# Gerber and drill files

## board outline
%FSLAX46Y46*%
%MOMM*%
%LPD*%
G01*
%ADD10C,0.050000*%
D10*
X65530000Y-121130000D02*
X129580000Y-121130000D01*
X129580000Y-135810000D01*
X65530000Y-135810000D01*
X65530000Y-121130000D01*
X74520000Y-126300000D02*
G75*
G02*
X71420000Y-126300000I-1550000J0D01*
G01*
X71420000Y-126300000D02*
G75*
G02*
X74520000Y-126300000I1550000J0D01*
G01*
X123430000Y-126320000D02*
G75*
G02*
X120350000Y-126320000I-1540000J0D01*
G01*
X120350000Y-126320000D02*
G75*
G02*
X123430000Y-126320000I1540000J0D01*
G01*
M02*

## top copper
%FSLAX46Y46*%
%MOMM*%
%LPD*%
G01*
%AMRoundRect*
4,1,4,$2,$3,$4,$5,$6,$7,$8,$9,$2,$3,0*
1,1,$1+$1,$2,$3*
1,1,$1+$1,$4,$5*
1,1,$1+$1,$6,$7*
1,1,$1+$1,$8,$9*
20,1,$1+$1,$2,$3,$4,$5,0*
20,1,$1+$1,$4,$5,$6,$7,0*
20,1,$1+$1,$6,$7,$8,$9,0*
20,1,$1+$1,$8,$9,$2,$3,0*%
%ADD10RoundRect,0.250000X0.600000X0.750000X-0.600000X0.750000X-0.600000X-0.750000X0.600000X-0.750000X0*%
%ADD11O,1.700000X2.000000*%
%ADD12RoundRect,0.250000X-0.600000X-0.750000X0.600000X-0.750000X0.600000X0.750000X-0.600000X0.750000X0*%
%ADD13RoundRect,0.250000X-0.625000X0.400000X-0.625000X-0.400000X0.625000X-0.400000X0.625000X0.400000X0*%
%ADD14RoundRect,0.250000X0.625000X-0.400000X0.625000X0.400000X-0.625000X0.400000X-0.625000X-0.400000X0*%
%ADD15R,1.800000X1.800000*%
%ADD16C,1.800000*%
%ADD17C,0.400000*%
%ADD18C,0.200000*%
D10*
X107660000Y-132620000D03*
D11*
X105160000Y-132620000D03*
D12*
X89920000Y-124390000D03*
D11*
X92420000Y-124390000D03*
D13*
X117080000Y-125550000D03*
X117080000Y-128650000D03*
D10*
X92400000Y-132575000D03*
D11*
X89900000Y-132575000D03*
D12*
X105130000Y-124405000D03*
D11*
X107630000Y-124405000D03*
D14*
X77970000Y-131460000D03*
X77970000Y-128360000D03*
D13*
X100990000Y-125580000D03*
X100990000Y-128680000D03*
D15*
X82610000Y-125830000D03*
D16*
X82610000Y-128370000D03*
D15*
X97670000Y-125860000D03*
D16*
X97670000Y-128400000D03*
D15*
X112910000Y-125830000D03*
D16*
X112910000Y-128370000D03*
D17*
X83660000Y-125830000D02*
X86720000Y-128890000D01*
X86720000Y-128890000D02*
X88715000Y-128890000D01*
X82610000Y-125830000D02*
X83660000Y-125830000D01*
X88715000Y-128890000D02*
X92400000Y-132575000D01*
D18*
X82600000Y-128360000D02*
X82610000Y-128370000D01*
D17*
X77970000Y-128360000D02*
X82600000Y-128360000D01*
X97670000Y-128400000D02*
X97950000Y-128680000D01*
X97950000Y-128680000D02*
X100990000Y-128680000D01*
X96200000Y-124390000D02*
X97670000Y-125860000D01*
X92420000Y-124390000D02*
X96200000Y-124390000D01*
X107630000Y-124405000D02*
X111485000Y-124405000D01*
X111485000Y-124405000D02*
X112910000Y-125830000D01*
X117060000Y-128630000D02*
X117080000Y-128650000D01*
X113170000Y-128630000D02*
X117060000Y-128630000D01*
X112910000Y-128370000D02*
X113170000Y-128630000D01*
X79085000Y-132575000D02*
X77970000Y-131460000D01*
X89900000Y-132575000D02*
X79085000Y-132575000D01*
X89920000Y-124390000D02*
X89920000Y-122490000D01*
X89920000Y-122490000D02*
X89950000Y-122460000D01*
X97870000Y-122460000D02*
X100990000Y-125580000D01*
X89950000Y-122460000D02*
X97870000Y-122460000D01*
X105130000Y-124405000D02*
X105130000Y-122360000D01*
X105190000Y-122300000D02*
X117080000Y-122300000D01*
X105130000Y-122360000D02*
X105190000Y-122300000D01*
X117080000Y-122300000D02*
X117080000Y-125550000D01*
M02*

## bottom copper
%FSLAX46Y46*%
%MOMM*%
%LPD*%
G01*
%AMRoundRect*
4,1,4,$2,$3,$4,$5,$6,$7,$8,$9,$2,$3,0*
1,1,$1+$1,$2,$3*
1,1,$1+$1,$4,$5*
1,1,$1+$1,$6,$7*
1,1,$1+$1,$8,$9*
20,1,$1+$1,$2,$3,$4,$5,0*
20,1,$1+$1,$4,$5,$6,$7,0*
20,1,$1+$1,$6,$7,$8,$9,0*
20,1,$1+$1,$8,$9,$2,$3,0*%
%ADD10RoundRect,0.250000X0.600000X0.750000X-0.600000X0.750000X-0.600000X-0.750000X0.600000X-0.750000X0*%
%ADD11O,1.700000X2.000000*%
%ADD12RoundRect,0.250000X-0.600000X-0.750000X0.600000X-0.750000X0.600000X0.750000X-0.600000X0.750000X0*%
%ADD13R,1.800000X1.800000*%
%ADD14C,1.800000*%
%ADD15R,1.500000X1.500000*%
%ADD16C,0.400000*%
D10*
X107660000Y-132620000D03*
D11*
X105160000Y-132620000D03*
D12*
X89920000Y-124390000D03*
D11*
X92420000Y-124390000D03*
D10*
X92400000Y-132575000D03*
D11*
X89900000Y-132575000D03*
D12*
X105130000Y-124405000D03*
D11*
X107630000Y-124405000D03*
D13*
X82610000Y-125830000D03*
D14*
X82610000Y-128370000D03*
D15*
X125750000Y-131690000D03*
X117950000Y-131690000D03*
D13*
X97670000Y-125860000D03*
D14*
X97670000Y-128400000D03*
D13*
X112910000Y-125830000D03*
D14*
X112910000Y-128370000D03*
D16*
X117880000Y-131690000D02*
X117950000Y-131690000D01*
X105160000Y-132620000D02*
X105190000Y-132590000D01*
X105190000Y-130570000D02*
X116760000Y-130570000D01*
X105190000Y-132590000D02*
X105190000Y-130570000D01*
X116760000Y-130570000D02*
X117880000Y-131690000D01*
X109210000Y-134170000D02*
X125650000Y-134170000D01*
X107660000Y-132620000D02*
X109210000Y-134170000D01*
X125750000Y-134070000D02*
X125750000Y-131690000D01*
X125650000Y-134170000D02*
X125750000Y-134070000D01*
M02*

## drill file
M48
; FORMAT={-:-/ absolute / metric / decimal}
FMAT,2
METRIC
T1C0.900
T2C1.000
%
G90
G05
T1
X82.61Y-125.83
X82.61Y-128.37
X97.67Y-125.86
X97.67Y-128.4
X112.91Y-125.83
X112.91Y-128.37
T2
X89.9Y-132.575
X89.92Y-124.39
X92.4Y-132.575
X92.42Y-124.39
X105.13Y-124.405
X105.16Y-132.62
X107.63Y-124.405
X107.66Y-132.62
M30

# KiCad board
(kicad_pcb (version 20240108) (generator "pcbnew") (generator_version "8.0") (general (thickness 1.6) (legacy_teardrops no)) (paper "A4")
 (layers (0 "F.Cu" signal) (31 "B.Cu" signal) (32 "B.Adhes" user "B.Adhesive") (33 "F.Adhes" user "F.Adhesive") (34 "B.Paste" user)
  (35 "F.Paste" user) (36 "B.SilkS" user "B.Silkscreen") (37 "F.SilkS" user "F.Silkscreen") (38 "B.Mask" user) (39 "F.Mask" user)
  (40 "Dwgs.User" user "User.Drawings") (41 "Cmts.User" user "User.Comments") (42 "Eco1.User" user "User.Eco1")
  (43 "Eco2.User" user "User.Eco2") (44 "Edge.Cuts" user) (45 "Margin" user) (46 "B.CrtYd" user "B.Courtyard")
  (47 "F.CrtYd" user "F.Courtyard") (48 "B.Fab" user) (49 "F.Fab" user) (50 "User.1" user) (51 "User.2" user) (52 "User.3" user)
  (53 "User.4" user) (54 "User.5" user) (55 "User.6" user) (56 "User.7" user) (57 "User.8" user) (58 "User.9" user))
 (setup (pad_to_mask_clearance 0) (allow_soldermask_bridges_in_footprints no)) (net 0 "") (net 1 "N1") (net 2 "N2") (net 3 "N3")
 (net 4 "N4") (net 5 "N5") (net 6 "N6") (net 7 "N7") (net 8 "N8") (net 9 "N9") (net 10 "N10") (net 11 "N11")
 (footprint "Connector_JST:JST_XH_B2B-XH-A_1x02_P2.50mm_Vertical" (layer "F.Cu") (at 107.66 132.62 180)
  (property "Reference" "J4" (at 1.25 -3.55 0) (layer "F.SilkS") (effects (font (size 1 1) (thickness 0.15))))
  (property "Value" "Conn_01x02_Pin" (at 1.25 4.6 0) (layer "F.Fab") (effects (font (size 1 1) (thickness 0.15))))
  (pad "1" thru_hole roundrect (at 0 0 180) (size 1.7 2) (drill 1) (layers "*.Cu" "*.Mask") (remove_unused_layers no)
   (roundrect_rratio 0.147059) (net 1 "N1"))
  (pad "2" thru_hole oval (at 2.5 0 180) (size 1.7 2) (drill 1) (layers "*.Cu" "*.Mask") (remove_unused_layers no) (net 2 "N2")))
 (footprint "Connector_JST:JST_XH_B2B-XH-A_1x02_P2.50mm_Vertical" (layer "F.Cu") (at 89.92 124.39)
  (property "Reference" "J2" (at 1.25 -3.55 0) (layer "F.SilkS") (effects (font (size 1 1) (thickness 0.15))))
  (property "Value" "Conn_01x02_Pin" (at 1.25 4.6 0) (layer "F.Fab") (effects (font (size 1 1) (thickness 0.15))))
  (pad "1" thru_hole roundrect (at 0 0) (size 1.7 2) (drill 1) (layers "*.Cu" "*.Mask") (remove_unused_layers no)
   (roundrect_rratio 0.147059) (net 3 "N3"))
  (pad "2" thru_hole oval (at 2.5 0) (size 1.7 2) (drill 1) (layers "*.Cu" "*.Mask") (remove_unused_layers no) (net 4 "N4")))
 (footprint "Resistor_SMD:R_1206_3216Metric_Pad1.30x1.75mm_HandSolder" (layer "F.Cu") (at 117.08 127.1 -90)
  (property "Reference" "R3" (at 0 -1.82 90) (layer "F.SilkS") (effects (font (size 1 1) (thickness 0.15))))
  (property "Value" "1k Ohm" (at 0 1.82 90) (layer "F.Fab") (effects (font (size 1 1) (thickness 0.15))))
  (pad "1" smd roundrect (at -1.55 0 270) (size 1.3 1.75) (layers "F.Cu" "F.Paste" "F.Mask") (roundrect_rratio 0.192308) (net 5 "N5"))
  (pad "2" smd roundrect (at 1.55 0 270) (size 1.3 1.75) (layers "F.Cu" "F.Paste" "F.Mask") (roundrect_rratio 0.192308) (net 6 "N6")))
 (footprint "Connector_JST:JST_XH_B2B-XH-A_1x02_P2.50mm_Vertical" (layer "F.Cu") (at 92.4 132.575 180)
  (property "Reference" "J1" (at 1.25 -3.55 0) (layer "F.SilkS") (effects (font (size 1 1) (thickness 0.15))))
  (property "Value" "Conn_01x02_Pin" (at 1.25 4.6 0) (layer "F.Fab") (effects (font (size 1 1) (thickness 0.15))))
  (pad "1" thru_hole roundrect (at 0 0 180) (size 1.7 2) (drill 1) (layers "*.Cu" "*.Mask") (remove_unused_layers no)
   (roundrect_rratio 0.147059) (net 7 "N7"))
  (pad "2" thru_hole oval (at 2.5 0 180) (size 1.7 2) (drill 1) (layers "*.Cu" "*.Mask") (remove_unused_layers no) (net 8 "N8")))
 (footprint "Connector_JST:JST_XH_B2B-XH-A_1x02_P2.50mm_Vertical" (layer "F.Cu") (at 105.13 124.405)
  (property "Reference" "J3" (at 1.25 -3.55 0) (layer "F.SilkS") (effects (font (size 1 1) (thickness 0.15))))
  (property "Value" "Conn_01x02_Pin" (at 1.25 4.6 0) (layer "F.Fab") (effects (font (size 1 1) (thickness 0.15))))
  (pad "1" thru_hole roundrect (at 0 0) (size 1.7 2) (drill 1) (layers "*.Cu" "*.Mask") (remove_unused_layers no)
   (roundrect_rratio 0.147059) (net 5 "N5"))
  (pad "2" thru_hole oval (at 2.5 0) (size 1.7 2) (drill 1) (layers "*.Cu" "*.Mask") (remove_unused_layers no) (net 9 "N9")))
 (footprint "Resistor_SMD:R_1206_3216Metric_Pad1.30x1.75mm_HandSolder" (layer "F.Cu") (at 77.97 129.91 90)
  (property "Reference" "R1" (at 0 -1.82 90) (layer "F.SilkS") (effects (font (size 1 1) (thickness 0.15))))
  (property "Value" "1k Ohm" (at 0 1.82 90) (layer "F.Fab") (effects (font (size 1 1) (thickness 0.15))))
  (pad "1" smd roundrect (at -1.55 0 90) (size 1.3 1.75) (layers "F.Cu" "F.Paste" "F.Mask") (roundrect_rratio 0.192308) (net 8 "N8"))
  (pad "2" smd roundrect (at 1.55 0 90) (size 1.3 1.75) (layers "F.Cu" "F.Paste" "F.Mask") (roundrect_rratio 0.192308) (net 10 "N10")))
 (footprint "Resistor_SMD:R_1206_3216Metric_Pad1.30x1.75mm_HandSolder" (layer "F.Cu") (at 100.99 127.13 -90)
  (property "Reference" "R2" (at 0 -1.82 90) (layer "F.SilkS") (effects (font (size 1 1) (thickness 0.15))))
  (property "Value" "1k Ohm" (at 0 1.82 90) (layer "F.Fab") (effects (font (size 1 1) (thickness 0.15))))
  (pad "1" smd roundrect (at -1.55 0 270) (size 1.3 1.75) (layers "F.Cu" "F.Paste" "F.Mask") (roundrect_rratio 0.192308) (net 3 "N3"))
  (pad "2" smd roundrect (at 1.55 0 270) (size 1.3 1.75) (layers "F.Cu" "F.Paste" "F.Mask") (roundrect_rratio 0.192308) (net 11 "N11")))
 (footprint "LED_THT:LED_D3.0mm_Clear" (layer "B.Cu") (at 82.61 125.83 -90)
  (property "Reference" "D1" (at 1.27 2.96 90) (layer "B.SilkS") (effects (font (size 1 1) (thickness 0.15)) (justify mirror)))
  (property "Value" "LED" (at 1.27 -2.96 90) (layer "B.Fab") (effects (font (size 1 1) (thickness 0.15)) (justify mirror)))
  (pad "1" thru_hole rect (at 0 0 270) (size 1.8 1.8) (drill 0.9) (layers "*.Cu" "*.Mask") (remove_unused_layers no) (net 7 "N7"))
  (pad "2" thru_hole circle (at 2.54 0 270) (size 1.8 1.8) (drill 0.9) (layers "*.Cu" "*.Mask") (remove_unused_layers no) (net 10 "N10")))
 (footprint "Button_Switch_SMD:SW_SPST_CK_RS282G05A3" (layer "B.Cu") (at 121.85 131.69 180)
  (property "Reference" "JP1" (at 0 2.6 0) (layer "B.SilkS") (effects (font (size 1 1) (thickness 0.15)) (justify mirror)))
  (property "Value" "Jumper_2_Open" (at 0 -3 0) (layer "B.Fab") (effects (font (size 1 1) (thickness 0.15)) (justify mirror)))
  (pad "1" smd rect (at -3.9 0 180) (size 1.5 1.5) (layers "B.Cu" "B.Paste" "B.Mask") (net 1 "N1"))
  (pad "2" smd rect (at 3.9 0 180) (size 1.5 1.5) (layers "B.Cu" "B.Paste" "B.Mask") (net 2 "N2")))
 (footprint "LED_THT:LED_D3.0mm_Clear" (layer "B.Cu") (at 97.67 125.86 -90)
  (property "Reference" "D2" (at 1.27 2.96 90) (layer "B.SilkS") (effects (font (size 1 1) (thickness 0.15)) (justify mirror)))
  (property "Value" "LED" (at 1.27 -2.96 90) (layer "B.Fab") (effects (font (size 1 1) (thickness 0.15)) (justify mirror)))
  (pad "1" thru_hole rect (at 0 0 270) (size 1.8 1.8) (drill 0.9) (layers "*.Cu" "*.Mask") (remove_unused_layers no) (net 4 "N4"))
  (pad "2" thru_hole circle (at 2.54 0 270) (size 1.8 1.8) (drill 0.9) (layers "*.Cu" "*.Mask") (remove_unused_layers no) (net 11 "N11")))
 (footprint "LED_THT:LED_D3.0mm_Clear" (layer "B.Cu") (at 112.91 125.83 -90)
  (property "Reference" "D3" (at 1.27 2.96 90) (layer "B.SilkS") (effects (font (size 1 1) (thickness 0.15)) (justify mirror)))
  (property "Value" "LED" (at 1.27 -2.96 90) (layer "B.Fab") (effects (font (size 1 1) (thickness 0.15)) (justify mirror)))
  (pad "1" thru_hole rect (at 0 0 270) (size 1.8 1.8) (drill 0.9) (layers "*.Cu" "*.Mask") (remove_unused_layers no) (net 9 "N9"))
  (pad "2" thru_hole circle (at 2.54 0 270) (size 1.8 1.8) (drill 0.9) (layers "*.Cu" "*.Mask") (remove_unused_layers no) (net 6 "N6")))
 (gr_rect (start 65.53 121.13) (end 129.58 135.81) (stroke (width 0.05) (type default)) (fill none) (layer "Edge.Cuts"))
 (gr_circle (center 72.97 126.3) (end 74.52 126.3) (stroke (width 0.05) (type default)) (fill none) (layer "Edge.Cuts"))
 (gr_circle (center 121.89 126.32) (end 123.43 126.32) (stroke (width 0.05) (type default)) (fill none) (layer "Edge.Cuts"))
 (segment (start 83.66 125.83) (end 86.72 128.89) (width 0.4) (layer "F.Cu") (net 7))
 (segment (start 86.72 128.89) (end 88.715 128.89) (width 0.4) (layer "F.Cu") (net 7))
 (segment (start 82.61 125.83) (end 83.66 125.83) (width 0.4) (layer "F.Cu") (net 7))
 (segment (start 88.715 128.89) (end 92.4 132.575) (width 0.4) (layer "F.Cu") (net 7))
 (segment (start 82.6 128.36) (end 82.61 128.37) (width 0.2) (layer "F.Cu") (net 10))
 (segment (start 77.97 128.36) (end 82.6 128.36) (width 0.4) (layer "F.Cu") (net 10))
 (segment (start 97.67 128.4) (end 97.95 128.68) (width 0.4) (layer "F.Cu") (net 11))
 (segment (start 97.95 128.68) (end 100.99 128.68) (width 0.4) (layer "F.Cu") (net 11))
 (segment (start 96.2 124.39) (end 97.67 125.86) (width 0.4) (layer "F.Cu") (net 4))
 (segment (start 92.42 124.39) (end 96.2 124.39) (width 0.4) (layer "F.Cu") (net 4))
 (segment (start 107.63 124.405) (end 111.485 124.405) (width 0.4) (layer "F.Cu") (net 9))
 (segment (start 111.485 124.405) (end 112.91 125.83) (width 0.4) (layer "F.Cu") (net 9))
 (segment (start 117.06 128.63) (end 117.08 128.65) (width 0.4) (layer "F.Cu") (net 6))
 (segment (start 113.17 128.63) (end 117.06 128.63) (width 0.4) (layer "F.Cu") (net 6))
 (segment (start 112.91 128.37) (end 113.17 128.63) (width 0.4) (layer "F.Cu") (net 6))
 (segment (start 79.085 132.575) (end 77.97 131.46) (width 0.4) (layer "F.Cu") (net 8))
 (segment (start 89.9 132.575) (end 79.085 132.575) (width 0.4) (layer "F.Cu") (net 8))
 (segment (start 89.92 124.39) (end 89.92 122.49) (width 0.4) (layer "F.Cu") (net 3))
 (segment (start 89.92 122.49) (end 89.95 122.46) (width 0.4) (layer "F.Cu") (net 3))
 (segment (start 97.87 122.46) (end 100.99 125.58) (width 0.4) (layer "F.Cu") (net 3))
 (segment (start 89.95 122.46) (end 97.87 122.46) (width 0.4) (layer "F.Cu") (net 3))
 (segment (start 105.13 124.405) (end 105.13 122.36) (width 0.4) (layer "F.Cu") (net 5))
 (segment (start 105.19 122.3) (end 117.08 122.3) (width 0.4) (layer "F.Cu") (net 5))
 (segment (start 105.13 122.36) (end 105.19 122.3) (width 0.4) (layer "F.Cu") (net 5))
 (segment (start 117.08 122.3) (end 117.08 125.55) (width 0.4) (layer "F.Cu") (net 5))
 (segment (start 117.88 131.69) (end 117.95 131.69) (width 0.4) (layer "B.Cu") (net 2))
 (segment (start 105.16 132.62) (end 105.19 132.59) (width 0.4) (layer "B.Cu") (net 2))
 (segment (start 105.19 130.57) (end 116.76 130.57) (width 0.4) (layer "B.Cu") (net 2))
 (segment (start 105.19 132.59) (end 105.19 130.57) (width 0.4) (layer "B.Cu") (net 2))
 (segment (start 116.76 130.57) (end 117.88 131.69) (width 0.4) (layer "B.Cu") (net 2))
 (segment (start 109.21 134.17) (end 125.65 134.17) (width 0.4) (layer "B.Cu") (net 1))
 (segment (start 107.66 132.62) (end 109.21 134.17) (width 0.4) (layer "B.Cu") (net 1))
 (segment (start 125.75 134.07) (end 125.75 131.69) (width 0.4) (layer "B.Cu") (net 1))
 (segment (start 125.65 134.17) (end 125.75 134.07) (width 0.4) (layer "B.Cu") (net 1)))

